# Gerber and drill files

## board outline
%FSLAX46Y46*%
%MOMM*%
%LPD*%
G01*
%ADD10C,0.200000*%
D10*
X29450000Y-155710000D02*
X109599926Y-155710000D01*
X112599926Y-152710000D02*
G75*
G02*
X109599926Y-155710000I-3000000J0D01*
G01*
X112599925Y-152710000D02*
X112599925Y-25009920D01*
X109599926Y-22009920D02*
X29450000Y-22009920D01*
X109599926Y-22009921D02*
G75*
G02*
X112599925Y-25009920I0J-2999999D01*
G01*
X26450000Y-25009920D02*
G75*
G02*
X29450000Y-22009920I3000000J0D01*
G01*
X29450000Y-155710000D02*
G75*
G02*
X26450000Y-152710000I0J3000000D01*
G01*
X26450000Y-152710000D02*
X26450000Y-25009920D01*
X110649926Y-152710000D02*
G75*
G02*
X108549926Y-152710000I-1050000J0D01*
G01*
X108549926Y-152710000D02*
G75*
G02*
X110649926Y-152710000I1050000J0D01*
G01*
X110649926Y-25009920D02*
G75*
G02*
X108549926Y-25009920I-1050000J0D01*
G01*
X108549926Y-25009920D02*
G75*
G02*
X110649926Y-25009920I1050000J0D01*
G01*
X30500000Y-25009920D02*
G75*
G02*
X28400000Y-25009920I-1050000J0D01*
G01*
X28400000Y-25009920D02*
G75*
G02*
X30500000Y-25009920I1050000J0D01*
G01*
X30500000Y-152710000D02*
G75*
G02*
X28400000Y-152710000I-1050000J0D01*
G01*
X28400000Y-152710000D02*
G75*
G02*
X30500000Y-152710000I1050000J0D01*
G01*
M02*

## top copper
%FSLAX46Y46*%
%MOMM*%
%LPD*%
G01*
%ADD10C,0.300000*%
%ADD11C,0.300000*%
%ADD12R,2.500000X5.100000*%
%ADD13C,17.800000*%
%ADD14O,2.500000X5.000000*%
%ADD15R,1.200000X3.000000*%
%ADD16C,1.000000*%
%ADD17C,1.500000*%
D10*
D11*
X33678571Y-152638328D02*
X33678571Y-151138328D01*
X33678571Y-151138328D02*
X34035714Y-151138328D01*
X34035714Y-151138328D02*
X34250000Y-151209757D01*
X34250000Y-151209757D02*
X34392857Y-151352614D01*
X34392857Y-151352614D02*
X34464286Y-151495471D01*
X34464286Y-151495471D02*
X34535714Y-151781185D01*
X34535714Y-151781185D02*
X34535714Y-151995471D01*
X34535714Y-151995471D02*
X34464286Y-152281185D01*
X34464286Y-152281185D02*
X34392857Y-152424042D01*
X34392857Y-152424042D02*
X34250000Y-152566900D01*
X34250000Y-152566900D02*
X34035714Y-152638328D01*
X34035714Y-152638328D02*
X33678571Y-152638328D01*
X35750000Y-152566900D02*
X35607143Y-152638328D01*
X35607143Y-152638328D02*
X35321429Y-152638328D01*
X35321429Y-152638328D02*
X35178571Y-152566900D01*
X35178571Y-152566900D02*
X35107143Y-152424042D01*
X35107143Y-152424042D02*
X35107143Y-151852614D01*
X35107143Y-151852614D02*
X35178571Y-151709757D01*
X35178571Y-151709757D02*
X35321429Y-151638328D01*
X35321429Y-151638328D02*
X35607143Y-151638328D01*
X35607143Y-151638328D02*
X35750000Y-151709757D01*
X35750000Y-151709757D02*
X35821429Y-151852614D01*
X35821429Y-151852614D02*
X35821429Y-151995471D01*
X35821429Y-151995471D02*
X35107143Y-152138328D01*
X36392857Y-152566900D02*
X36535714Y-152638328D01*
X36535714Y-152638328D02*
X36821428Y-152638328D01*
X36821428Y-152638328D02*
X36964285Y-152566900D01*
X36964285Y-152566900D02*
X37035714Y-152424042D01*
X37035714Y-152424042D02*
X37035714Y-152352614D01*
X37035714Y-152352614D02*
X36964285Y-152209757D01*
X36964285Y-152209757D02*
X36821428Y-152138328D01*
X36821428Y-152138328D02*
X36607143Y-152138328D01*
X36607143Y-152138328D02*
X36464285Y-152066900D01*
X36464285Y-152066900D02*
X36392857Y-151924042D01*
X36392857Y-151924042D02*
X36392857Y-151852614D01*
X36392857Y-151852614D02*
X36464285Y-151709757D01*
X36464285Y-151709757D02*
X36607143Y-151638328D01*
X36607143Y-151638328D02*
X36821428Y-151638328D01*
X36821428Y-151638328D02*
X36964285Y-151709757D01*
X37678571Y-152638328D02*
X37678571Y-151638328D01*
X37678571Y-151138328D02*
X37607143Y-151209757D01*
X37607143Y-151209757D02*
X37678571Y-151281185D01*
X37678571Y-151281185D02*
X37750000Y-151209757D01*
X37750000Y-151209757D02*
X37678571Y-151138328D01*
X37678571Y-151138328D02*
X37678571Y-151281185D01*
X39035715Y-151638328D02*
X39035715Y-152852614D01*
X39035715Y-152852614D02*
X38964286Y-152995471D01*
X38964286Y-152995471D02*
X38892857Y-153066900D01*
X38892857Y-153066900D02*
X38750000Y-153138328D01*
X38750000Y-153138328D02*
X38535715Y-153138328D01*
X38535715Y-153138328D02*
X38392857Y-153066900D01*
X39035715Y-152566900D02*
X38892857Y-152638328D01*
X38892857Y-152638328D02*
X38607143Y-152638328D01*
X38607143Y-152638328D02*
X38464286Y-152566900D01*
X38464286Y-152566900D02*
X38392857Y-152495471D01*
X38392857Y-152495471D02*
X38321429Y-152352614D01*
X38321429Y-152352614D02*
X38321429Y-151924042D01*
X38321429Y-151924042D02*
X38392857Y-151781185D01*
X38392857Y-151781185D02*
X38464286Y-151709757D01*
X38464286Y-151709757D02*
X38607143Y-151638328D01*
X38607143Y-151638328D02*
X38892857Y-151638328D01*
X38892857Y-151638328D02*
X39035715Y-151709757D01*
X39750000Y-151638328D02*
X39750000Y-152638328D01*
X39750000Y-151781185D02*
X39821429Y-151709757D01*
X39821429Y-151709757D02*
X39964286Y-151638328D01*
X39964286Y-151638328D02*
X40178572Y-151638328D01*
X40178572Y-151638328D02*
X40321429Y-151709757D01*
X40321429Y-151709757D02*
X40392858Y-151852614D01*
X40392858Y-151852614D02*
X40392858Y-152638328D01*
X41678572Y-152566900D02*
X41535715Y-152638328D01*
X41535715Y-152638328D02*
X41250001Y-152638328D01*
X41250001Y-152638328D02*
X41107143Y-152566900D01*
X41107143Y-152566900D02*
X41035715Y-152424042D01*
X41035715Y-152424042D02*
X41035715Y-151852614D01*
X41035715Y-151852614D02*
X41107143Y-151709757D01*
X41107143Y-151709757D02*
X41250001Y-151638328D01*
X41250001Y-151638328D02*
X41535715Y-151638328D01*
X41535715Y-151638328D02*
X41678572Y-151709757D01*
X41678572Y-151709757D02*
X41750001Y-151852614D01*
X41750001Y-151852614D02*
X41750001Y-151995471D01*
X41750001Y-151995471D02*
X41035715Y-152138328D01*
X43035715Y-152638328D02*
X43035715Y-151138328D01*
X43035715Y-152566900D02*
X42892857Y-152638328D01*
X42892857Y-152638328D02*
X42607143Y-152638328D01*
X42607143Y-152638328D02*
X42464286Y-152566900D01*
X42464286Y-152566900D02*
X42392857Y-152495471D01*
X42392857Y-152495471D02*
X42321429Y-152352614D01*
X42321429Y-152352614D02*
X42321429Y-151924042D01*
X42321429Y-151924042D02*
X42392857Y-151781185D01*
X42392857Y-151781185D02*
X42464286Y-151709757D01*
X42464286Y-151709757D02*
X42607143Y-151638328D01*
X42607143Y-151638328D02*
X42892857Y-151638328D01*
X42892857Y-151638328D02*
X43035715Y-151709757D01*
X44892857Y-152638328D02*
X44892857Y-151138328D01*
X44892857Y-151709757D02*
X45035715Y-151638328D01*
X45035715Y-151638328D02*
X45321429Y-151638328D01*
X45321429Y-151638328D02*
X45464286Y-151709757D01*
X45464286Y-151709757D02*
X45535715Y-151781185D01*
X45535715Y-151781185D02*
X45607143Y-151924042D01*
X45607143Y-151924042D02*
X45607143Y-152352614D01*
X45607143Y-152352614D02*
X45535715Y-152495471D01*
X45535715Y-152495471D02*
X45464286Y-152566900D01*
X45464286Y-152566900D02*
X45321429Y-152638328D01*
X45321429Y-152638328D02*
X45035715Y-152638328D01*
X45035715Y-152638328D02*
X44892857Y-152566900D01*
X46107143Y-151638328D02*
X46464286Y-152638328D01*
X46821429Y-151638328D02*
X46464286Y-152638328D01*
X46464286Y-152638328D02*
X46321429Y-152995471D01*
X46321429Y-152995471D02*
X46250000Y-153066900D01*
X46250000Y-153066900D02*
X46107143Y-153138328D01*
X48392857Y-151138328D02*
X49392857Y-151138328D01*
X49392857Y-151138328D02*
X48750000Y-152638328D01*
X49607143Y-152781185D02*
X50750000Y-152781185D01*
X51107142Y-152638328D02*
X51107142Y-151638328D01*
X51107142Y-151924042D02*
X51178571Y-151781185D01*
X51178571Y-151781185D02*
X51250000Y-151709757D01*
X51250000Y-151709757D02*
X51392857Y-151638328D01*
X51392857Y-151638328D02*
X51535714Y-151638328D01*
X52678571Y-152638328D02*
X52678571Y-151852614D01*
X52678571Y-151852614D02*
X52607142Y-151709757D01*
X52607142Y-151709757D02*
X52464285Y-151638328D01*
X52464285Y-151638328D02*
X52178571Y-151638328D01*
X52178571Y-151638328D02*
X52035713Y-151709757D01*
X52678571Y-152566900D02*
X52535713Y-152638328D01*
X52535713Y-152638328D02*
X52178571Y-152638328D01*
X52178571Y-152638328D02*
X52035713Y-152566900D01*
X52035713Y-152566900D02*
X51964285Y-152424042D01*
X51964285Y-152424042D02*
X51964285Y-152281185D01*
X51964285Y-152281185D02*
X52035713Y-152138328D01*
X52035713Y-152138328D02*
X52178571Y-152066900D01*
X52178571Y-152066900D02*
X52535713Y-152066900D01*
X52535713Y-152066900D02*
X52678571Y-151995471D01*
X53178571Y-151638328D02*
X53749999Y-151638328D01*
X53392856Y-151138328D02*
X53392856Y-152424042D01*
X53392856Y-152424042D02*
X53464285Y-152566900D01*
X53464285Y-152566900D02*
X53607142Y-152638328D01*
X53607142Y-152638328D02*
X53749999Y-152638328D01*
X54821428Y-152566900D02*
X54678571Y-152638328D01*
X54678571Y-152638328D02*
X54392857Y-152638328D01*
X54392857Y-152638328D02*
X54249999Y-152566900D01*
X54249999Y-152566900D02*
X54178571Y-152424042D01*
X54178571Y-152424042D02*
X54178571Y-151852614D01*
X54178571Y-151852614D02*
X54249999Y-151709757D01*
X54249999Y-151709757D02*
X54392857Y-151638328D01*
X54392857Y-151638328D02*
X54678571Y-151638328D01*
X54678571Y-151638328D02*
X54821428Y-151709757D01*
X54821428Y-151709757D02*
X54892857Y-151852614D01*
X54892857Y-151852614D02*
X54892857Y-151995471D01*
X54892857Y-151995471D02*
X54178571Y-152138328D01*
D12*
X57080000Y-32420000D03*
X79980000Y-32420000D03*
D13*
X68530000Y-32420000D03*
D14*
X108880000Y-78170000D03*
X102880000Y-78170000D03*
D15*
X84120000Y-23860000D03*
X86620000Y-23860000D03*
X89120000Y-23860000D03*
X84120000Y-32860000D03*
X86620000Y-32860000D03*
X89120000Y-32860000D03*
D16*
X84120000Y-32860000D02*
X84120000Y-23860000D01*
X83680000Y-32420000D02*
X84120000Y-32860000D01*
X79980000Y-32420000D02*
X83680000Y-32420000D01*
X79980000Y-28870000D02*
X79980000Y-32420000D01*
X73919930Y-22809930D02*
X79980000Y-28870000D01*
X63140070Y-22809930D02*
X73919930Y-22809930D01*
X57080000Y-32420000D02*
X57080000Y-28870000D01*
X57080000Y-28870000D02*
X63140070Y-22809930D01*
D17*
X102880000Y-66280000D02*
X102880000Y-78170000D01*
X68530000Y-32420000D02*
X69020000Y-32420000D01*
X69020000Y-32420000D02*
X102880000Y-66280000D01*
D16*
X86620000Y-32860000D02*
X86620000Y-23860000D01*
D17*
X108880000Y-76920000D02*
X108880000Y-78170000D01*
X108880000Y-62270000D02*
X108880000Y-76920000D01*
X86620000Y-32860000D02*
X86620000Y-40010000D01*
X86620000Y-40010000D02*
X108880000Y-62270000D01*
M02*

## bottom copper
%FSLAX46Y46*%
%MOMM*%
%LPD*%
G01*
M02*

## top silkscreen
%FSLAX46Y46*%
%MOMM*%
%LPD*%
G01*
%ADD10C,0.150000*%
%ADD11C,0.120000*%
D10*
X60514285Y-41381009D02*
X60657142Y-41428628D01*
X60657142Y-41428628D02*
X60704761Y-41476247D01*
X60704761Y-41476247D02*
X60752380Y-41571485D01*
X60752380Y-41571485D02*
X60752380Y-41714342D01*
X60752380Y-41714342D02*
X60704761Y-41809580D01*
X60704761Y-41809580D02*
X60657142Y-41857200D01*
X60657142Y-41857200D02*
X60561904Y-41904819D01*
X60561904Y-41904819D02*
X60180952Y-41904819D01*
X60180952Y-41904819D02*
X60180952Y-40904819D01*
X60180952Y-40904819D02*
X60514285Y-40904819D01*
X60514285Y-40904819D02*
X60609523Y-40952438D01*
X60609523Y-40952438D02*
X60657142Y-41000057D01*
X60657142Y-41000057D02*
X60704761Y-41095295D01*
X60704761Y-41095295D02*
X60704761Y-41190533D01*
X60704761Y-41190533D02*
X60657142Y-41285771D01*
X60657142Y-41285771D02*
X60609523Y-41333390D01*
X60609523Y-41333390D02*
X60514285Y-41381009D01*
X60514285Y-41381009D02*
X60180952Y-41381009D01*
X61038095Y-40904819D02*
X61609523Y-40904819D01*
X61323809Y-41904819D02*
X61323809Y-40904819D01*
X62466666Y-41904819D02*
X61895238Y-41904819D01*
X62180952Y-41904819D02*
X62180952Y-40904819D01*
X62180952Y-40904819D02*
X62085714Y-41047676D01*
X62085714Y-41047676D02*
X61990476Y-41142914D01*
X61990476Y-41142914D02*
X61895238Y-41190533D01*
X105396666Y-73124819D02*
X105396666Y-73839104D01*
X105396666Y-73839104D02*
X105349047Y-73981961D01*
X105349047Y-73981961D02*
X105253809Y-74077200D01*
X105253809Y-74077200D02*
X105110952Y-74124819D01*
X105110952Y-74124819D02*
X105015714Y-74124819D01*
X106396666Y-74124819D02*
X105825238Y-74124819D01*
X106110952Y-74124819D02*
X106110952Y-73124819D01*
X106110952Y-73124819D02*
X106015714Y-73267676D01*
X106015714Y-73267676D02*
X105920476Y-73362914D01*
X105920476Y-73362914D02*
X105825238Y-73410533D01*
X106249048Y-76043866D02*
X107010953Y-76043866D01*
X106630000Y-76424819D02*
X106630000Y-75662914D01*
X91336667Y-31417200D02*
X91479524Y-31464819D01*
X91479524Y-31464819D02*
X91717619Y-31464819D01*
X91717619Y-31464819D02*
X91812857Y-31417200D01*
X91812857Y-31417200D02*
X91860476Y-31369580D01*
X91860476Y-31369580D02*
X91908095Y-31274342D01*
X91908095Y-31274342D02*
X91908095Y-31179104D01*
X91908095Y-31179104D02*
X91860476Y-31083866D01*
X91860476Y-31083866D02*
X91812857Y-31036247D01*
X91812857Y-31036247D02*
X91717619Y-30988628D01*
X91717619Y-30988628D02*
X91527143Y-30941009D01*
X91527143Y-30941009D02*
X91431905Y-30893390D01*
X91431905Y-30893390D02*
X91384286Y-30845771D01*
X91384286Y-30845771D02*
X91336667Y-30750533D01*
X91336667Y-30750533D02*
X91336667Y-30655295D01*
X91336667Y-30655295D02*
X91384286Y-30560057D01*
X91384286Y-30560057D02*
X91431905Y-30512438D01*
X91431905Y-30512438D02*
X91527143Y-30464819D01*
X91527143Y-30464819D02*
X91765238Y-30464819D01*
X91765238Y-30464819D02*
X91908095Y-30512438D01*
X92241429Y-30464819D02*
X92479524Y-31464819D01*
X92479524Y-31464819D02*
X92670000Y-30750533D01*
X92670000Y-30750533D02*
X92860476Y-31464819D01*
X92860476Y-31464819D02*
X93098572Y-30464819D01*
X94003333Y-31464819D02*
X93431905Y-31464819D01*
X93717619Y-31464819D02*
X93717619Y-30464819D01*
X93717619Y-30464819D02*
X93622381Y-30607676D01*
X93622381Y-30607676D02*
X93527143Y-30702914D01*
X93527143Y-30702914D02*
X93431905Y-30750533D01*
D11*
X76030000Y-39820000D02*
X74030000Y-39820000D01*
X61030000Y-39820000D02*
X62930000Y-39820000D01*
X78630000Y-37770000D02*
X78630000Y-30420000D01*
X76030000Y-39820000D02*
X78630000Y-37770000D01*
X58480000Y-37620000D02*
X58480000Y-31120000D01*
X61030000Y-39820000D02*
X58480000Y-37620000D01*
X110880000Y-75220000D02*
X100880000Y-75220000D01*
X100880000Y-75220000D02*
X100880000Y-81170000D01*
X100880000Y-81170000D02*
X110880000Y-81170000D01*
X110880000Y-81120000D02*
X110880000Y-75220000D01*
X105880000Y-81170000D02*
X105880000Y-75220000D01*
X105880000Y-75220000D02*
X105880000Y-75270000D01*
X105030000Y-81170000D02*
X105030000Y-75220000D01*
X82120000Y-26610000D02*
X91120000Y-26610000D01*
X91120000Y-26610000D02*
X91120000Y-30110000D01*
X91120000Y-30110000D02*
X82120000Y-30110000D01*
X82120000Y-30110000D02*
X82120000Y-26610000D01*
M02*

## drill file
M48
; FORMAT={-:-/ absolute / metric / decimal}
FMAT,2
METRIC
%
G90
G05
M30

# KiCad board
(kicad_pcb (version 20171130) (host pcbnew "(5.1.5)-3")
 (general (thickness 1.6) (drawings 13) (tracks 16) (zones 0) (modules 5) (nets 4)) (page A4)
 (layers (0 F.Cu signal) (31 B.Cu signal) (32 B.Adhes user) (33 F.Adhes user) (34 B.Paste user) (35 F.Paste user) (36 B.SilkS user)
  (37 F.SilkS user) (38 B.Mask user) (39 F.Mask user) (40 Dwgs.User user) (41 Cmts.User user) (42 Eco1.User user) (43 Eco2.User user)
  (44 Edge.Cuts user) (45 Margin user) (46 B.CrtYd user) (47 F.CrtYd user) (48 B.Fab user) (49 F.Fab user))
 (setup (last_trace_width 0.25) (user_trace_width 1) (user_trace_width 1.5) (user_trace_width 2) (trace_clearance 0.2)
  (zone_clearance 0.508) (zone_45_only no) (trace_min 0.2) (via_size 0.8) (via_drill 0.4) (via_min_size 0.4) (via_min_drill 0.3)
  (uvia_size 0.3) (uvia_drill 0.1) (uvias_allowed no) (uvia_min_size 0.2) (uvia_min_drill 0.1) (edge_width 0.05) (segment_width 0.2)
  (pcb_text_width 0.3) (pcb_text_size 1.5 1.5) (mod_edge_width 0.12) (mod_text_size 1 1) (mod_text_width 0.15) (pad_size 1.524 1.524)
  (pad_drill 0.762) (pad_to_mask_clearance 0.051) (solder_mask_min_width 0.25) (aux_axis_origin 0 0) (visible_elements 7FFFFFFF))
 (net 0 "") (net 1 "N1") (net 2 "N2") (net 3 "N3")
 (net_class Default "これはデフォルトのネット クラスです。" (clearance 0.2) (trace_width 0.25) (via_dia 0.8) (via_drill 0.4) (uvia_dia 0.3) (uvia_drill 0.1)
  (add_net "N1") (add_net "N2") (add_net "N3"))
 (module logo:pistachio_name (layer B.Cu) (at 52.1 145.21 180)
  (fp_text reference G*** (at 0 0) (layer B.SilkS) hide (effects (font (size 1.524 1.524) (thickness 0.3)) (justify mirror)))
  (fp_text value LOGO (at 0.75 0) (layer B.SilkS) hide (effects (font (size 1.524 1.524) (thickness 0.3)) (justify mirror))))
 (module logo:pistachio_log (layer B.Cu) (at 88.18 137.35 180)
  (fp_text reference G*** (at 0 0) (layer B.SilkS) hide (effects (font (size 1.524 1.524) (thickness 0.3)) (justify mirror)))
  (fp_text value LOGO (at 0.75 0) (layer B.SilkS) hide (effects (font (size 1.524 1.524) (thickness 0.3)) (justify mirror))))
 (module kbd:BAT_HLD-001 (layer F.Cu) (at 68.53 32.42 180)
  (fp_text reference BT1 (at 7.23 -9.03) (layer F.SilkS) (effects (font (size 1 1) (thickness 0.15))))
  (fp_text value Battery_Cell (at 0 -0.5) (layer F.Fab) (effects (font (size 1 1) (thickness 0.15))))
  (fp_line (start -7.5 -7.4) (end -5.5 -7.4) (layer F.SilkS) (width 0.12))
  (fp_line (start 7.5 -7.4) (end 5.6 -7.4) (layer F.SilkS) (width 0.12))
  (fp_line (start -10.1 -5.35) (end -10.1 2) (layer F.SilkS) (width 0.12))
  (fp_line (start -7.5 -7.4) (end -10.1 -5.35) (layer F.SilkS) (width 0.12))
  (fp_line (start 10.05 -5.2) (end 10.05 1.3) (layer F.SilkS) (width 0.12))
  (fp_line (start 7.5 -7.4) (end 10.05 -5.2) (layer F.SilkS) (width 0.12))
  (pad 1 smd rect (at 11.45 0 180) (size 2.5 5.1) (layers F.Cu F.Paste F.Mask) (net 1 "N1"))
  (pad 1 smd rect (at -11.45 0 180) (size 2.5 5.1) (layers F.Cu F.Paste F.Mask) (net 1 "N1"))
  (pad 2 smd circle (at 0 0 180) (size 17.8 17.8) (layers F.Cu F.Paste F.Mask) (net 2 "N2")))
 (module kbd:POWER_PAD (layer F.Cu) (at 105.88 78.17 180)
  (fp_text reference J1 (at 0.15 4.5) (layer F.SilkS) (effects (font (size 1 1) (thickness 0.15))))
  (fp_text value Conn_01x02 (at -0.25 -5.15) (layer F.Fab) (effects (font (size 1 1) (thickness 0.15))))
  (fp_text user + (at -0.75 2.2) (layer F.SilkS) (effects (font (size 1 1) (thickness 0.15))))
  (fp_line (start -5 2.95) (end 5 2.95) (layer F.SilkS) (width 0.12))
  (fp_line (start 5 2.95) (end 5 -3) (layer F.SilkS) (width 0.12))
  (fp_line (start 5 -3) (end -5 -3) (layer F.SilkS) (width 0.12))
  (fp_line (start -5 -2.95) (end -5 2.95) (layer F.SilkS) (width 0.12))
  (fp_line (start 0 -3) (end 0 2.95) (layer F.SilkS) (width 0.12))
  (fp_line (start 0 2.95) (end 0 2.9) (layer F.SilkS) (width 0.12))
  (fp_line (start 0.85 -3) (end 0.85 2.95) (layer F.SilkS) (width 0.12))
  (pad 1 smd oval (at -3 0 180) (size 2.5 5) (layers F.Cu F.Paste F.Mask) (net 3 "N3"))
  (pad 2 smd oval (at 3 0 180) (size 2.5 5) (layers F.Cu F.Paste F.Mask) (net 2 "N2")))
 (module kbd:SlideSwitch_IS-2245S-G (layer F.Cu) (at 86.62 28.36)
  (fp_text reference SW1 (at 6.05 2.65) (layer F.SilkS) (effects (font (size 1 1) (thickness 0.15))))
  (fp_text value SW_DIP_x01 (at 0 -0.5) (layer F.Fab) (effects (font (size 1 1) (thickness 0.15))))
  (fp_line (start -4.5 -1.75) (end 4.5 -1.75) (layer F.SilkS) (width 0.12))
  (fp_line (start 4.5 -1.75) (end 4.5 1.75) (layer F.SilkS) (width 0.12))
  (fp_line (start 4.5 1.75) (end -4.5 1.75) (layer F.SilkS) (width 0.12))
  (fp_line (start -4.5 1.75) (end -4.5 -1.75) (layer F.SilkS) (width 0.12))
  (pad 1 smd rect (at -2.5 -4.5) (size 1.2 3) (layers F.Cu F.Paste F.Mask) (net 1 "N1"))
  (pad 2 smd rect (at 0 -4.5) (size 1.2 3) (layers F.Cu F.Paste F.Mask) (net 3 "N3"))
  (pad 3 smd rect (at 2.5 -4.5) (size 1.2 3) (layers F.Cu F.Paste F.Mask))
  (pad 1 smd rect (at -2.5 4.5) (size 1.2 3) (layers F.Cu F.Paste F.Mask) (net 1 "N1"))
  (pad 2 smd rect (at 0 4.5) (size 1.2 3) (layers F.Cu F.Paste F.Mask) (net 3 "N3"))
  (pad 3 smd rect (at 2.5 4.5) (size 1.2 3) (layers F.Cu F.Paste F.Mask)))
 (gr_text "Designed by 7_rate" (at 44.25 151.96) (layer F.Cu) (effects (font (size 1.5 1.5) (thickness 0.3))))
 (gr_line (start 29.45 155.71) (end 109.599926 155.71) (layer Edge.Cuts) (width 0.2))
 (gr_arc (start 109.599926 152.71) (end 109.599926 155.71) (angle -90) (layer Edge.Cuts) (width 0.2))
 (gr_line (start 112.599925 152.71) (end 112.599925 25.00992) (layer Edge.Cuts) (width 0.2))
 (gr_line (start 109.599926 22.00992) (end 29.45 22.00992) (layer Edge.Cuts) (width 0.2))
 (gr_arc (start 109.599926 25.00992) (end 112.599925 25.00992) (angle -90) (layer Edge.Cuts) (width 0.2))
 (gr_arc (start 29.45 25.00992) (end 29.45 22.00992) (angle -90) (layer Edge.Cuts) (width 0.2))
 (gr_arc (start 29.45 152.71) (end 26.45 152.71) (angle -90) (layer Edge.Cuts) (width 0.2))
 (gr_line (start 26.45 152.71) (end 26.45 25.00992) (layer Edge.Cuts) (width 0.2))
 (gr_circle (center 109.599926 152.71) (end 110.649926 152.71) (layer Edge.Cuts) (width 0.2))
 (gr_circle (center 109.599926 25.00992) (end 110.649926 25.00992) (layer Edge.Cuts) (width 0.2))
 (gr_circle (center 29.45 25.00992) (end 30.5 25.00992) (layer Edge.Cuts) (width 0.2))
 (gr_circle (center 29.45 152.71) (end 30.5 152.71) (layer Edge.Cuts) (width 0.2))
 (segment (start 84.12 32.86) (end 84.12 23.86) (width 1) (layer F.Cu) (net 1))
 (segment (start 83.68 32.42) (end 84.12 32.86) (width 1) (layer F.Cu) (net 1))
 (segment (start 79.98 32.42) (end 83.68 32.42) (width 1) (layer F.Cu) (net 1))
 (segment (start 79.98 28.87) (end 79.98 32.42) (width 1) (layer F.Cu) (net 1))
 (segment (start 73.91993 22.80993) (end 79.98 28.87) (width 1) (layer F.Cu) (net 1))
 (segment (start 63.14007 22.80993) (end 73.91993 22.80993) (width 1) (layer F.Cu) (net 1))
 (segment (start 57.08 32.42) (end 57.08 28.87) (width 1) (layer F.Cu) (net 1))
 (segment (start 57.08 28.87) (end 63.14007 22.80993) (width 1) (layer F.Cu) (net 1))
 (segment (start 102.88 66.28) (end 102.88 78.17) (width 1.5) (layer F.Cu) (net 2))
 (segment (start 68.53 32.42) (end 69.02 32.42) (width 1.5) (layer F.Cu) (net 2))
 (segment (start 69.02 32.42) (end 102.88 66.28) (width 1.5) (layer F.Cu) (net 2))
 (segment (start 86.62 32.86) (end 86.62 23.86) (width 1) (layer F.Cu) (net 3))
 (segment (start 108.88 76.92) (end 108.88 78.17) (width 1.5) (layer F.Cu) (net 3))
 (segment (start 108.88 62.27) (end 108.88 76.92) (width 1.5) (layer F.Cu) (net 3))
 (segment (start 86.62 32.86) (end 86.62 40.01) (width 1.5) (layer F.Cu) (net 3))
 (segment (start 86.62 40.01) (end 108.88 62.27) (width 1.5) (layer F.Cu) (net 3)))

